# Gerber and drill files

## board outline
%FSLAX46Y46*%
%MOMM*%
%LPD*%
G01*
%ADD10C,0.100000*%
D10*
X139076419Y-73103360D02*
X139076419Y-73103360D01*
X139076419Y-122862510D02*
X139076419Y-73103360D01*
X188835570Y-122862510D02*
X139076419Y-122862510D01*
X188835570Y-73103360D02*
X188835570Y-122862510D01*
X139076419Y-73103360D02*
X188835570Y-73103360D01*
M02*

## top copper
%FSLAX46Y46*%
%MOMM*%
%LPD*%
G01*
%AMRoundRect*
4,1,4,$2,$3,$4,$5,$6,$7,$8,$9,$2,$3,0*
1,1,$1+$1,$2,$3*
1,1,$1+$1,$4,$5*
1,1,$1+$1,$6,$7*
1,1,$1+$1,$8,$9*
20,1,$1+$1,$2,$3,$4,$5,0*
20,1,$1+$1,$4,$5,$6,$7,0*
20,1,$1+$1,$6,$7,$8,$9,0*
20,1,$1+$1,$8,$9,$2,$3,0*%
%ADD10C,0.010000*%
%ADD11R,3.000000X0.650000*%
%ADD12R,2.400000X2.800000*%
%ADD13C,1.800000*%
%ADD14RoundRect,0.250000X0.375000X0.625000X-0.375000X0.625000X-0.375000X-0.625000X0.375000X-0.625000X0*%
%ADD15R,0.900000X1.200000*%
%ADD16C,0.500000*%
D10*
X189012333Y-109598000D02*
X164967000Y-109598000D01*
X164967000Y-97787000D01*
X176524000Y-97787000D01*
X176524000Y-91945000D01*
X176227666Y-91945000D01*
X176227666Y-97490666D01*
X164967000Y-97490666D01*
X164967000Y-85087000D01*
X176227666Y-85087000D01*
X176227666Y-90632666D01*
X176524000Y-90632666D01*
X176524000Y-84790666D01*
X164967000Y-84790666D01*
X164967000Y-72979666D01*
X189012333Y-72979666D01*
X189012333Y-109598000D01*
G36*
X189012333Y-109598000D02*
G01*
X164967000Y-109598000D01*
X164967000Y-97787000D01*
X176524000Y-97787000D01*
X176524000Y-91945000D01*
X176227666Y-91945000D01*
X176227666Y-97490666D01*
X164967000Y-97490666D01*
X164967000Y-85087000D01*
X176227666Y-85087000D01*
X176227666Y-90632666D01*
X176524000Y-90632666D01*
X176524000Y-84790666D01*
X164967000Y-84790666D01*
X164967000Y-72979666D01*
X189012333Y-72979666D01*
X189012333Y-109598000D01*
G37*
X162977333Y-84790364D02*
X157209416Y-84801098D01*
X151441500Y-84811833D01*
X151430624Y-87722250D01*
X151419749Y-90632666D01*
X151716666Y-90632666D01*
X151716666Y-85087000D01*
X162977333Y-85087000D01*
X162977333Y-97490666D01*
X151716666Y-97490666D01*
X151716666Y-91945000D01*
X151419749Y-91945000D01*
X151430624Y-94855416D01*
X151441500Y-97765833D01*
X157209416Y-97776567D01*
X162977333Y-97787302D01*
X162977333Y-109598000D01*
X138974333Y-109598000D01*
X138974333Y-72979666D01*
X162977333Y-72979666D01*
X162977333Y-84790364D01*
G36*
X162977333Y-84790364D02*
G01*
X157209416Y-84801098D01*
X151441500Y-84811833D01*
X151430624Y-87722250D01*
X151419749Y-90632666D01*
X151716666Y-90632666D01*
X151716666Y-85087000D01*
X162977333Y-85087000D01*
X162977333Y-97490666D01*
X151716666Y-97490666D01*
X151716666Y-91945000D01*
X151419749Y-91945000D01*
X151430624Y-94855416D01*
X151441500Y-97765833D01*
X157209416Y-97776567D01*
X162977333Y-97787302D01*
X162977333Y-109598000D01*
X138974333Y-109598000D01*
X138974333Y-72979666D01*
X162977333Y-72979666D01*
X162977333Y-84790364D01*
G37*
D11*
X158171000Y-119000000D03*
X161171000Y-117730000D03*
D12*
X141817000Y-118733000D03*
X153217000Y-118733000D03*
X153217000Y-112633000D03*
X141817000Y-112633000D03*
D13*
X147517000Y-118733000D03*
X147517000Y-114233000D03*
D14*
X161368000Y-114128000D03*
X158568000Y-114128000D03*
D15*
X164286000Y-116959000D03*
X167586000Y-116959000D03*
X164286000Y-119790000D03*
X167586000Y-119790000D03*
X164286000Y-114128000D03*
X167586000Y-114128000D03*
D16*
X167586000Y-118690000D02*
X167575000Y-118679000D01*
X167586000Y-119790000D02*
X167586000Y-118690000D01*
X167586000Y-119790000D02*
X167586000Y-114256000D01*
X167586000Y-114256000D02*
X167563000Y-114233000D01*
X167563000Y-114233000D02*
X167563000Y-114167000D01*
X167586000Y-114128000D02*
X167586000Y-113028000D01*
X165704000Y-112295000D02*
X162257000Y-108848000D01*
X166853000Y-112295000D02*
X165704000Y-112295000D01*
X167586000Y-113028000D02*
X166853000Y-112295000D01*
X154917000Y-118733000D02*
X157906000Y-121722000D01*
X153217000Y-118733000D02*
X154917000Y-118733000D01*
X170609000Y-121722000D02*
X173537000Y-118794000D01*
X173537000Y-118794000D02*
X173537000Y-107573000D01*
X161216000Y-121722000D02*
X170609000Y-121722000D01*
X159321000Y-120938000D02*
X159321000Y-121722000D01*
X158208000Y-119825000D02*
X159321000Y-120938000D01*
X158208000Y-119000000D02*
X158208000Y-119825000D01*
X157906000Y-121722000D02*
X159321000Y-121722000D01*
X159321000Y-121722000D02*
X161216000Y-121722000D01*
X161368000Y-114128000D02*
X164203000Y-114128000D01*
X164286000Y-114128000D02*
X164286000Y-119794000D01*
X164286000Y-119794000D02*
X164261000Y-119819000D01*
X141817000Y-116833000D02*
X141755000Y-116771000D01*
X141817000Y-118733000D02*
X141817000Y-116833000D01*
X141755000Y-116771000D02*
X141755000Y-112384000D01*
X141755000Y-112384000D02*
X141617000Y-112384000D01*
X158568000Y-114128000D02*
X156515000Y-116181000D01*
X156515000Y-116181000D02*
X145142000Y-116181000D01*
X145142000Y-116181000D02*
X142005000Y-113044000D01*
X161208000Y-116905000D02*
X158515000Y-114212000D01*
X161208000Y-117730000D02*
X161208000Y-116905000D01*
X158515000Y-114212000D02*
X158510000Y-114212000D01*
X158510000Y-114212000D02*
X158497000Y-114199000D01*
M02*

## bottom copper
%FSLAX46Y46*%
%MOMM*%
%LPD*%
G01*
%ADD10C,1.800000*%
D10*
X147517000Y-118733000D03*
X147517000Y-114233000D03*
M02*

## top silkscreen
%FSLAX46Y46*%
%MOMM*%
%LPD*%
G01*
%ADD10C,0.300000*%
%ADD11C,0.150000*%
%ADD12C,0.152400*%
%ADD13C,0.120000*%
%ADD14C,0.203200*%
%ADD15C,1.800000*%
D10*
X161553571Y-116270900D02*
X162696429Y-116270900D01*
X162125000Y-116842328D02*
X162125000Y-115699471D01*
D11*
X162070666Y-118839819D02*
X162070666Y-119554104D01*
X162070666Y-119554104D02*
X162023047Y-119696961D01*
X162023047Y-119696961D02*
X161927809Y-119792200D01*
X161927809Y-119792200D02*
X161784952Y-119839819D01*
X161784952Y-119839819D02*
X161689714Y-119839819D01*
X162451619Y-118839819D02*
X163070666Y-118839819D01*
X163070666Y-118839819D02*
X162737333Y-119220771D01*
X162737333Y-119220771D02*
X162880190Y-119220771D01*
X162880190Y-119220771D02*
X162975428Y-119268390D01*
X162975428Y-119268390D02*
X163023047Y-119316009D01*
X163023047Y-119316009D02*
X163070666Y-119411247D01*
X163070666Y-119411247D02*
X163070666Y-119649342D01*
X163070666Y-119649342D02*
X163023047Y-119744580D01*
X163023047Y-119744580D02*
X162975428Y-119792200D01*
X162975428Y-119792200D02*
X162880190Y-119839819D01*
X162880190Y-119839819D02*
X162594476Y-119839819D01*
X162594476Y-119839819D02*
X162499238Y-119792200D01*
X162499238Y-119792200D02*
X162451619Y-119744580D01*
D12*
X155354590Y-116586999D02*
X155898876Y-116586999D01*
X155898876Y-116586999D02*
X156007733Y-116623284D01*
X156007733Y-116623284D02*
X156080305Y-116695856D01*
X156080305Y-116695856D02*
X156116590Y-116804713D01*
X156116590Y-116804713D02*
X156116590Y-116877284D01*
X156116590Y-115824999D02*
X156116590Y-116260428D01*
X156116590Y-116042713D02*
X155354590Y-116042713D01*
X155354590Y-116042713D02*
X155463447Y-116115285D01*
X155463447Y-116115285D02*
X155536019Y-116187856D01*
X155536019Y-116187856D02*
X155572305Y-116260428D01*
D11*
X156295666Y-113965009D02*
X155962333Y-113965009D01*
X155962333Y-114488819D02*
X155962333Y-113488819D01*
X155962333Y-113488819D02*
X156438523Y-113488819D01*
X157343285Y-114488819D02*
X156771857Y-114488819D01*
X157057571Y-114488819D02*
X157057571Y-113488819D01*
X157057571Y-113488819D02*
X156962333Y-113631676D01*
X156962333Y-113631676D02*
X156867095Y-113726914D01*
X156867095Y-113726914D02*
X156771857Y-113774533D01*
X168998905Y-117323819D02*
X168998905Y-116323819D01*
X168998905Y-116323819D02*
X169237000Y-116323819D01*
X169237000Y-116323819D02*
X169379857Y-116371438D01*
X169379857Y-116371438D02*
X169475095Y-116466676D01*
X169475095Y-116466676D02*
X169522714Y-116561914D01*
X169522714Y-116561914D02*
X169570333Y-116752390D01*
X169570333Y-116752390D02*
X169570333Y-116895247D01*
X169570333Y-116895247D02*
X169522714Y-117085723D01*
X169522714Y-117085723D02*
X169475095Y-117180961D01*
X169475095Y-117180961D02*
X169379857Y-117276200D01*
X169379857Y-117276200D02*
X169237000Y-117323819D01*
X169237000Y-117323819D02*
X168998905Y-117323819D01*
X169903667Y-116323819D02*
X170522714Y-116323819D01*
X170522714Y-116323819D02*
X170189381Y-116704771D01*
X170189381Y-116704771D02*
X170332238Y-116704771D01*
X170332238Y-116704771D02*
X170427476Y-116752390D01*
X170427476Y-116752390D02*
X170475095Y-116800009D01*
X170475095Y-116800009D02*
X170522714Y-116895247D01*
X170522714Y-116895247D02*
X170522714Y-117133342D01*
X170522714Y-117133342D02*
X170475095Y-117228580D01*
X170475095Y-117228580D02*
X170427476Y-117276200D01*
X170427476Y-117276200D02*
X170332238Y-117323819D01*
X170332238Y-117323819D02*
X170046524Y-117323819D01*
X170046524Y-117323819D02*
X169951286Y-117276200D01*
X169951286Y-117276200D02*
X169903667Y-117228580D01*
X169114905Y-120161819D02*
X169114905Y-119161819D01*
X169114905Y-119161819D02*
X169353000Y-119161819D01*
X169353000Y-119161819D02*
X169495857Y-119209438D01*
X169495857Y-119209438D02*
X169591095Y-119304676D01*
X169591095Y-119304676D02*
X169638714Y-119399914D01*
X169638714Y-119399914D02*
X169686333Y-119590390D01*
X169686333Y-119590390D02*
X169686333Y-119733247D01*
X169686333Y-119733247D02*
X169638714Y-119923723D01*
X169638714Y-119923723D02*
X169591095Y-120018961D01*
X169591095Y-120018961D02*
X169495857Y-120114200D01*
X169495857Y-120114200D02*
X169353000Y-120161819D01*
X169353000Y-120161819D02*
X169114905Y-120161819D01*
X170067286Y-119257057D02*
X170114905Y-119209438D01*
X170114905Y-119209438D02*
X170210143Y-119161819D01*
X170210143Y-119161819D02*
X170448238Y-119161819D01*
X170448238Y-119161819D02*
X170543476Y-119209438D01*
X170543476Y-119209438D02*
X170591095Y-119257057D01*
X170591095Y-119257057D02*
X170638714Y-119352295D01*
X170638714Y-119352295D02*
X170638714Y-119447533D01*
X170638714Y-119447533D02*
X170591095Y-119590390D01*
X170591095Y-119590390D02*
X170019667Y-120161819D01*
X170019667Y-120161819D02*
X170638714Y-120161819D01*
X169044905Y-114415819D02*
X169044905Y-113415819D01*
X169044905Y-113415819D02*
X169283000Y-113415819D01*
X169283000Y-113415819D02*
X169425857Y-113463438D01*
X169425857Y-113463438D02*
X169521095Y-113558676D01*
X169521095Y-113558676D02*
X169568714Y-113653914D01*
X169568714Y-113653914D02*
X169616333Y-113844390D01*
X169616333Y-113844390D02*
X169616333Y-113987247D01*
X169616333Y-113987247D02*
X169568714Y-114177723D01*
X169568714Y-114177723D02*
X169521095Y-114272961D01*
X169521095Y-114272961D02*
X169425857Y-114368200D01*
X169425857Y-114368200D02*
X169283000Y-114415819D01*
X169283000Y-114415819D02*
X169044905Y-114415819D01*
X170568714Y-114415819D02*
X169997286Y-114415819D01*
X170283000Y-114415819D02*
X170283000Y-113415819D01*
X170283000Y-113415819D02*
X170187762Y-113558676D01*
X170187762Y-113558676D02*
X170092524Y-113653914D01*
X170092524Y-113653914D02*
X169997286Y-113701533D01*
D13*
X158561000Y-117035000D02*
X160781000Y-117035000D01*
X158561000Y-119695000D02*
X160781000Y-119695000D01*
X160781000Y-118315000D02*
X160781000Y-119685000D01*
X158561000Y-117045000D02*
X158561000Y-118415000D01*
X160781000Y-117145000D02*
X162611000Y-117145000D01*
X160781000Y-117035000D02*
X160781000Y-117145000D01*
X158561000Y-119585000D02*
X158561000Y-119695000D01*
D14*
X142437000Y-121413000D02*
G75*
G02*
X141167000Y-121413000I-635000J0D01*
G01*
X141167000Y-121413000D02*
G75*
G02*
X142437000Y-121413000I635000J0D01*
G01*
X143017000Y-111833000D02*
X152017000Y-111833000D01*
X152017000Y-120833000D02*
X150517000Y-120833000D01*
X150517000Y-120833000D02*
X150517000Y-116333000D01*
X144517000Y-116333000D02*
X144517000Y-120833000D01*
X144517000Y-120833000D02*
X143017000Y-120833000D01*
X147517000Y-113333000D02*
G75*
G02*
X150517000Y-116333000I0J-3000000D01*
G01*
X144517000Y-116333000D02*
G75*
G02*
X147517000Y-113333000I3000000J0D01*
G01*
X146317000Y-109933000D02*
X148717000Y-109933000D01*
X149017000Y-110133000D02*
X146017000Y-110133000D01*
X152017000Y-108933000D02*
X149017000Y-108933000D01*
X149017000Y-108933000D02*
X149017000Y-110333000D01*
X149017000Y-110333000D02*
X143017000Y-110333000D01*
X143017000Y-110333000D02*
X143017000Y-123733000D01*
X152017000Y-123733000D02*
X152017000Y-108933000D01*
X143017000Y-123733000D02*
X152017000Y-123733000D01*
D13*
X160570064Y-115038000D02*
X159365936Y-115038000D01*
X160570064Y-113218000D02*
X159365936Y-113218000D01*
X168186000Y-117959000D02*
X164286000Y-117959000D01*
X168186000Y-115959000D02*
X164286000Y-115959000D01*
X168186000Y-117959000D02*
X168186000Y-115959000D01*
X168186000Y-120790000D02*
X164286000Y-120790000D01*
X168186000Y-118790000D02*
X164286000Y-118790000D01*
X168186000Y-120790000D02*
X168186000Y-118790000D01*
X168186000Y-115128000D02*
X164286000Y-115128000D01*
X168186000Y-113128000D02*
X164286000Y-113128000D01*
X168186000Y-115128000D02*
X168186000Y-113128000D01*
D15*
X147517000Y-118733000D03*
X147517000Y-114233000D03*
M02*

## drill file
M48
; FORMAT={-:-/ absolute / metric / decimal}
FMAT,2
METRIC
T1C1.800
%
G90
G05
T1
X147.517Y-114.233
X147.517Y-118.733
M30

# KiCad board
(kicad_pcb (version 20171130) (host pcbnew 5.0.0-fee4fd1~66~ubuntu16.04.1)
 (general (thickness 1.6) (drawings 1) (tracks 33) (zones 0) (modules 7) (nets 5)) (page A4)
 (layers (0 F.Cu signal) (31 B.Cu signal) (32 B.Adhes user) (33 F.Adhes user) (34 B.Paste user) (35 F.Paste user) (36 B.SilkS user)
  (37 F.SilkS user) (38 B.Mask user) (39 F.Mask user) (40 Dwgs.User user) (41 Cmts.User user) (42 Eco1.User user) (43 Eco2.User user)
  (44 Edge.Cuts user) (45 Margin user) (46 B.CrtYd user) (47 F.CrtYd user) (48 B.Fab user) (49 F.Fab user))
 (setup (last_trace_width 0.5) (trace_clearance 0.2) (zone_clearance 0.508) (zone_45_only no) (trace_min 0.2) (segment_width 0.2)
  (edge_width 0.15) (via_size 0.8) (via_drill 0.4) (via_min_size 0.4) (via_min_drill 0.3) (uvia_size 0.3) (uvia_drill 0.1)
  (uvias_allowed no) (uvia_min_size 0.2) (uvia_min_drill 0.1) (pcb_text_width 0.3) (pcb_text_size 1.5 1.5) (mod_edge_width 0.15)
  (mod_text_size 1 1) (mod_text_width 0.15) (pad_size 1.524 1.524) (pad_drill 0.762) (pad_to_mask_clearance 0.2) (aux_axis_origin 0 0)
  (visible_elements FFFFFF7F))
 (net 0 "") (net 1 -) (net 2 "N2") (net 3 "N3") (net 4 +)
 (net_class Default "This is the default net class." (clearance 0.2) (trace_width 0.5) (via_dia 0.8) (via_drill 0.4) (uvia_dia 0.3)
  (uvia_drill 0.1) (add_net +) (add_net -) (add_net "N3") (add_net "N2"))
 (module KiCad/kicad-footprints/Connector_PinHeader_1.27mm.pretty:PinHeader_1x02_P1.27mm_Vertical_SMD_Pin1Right (layer F.Cu)
  (at 159.671 118.365)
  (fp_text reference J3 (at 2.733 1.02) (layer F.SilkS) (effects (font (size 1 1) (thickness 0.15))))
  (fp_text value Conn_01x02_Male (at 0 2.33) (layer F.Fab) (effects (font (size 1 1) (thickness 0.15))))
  (fp_line (start -1.11 -1.33) (end 1.11 -1.33) (layer F.SilkS) (width 0.12))
  (fp_line (start -1.11 1.33) (end 1.11 1.33) (layer F.SilkS) (width 0.12))
  (fp_line (start 1.11 -0.05) (end 1.11 1.32) (layer F.SilkS) (width 0.12))
  (fp_line (start -1.11 -1.32) (end -1.11 0.05) (layer F.SilkS) (width 0.12))
  (fp_line (start 1.11 -1.22) (end 2.94 -1.22) (layer F.SilkS) (width 0.12))
  (fp_line (start 1.11 -1.33) (end 1.11 -1.22) (layer F.SilkS) (width 0.12))
  (fp_line (start -1.11 1.22) (end -1.11 1.33) (layer F.SilkS) (width 0.12))
  (pad 2 smd rect (at -1.5 0.635) (size 3 0.65) (layers F.Cu F.Paste F.Mask) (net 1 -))
  (pad 1 smd rect (at 1.5 -0.635) (size 3 0.65) (layers F.Cu F.Paste F.Mask) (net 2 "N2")))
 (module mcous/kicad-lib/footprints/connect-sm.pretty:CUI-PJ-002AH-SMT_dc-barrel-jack (layer F.Cu) (at 147.517 116.333 90)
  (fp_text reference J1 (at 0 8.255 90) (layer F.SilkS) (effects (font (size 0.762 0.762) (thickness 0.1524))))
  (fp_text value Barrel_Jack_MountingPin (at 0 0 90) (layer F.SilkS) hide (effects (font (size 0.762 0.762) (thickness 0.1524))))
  (fp_circle (center -5.08 -5.715) (end -4.445 -5.715) (layer F.SilkS) (width 0.2032))
  (fp_line (start 4.5 -4.5) (end 4.5 4.5) (layer F.SilkS) (width 0.2032))
  (fp_line (start -4.5 4.5) (end -4.5 3) (layer F.SilkS) (width 0.2032))
  (fp_line (start -4.5 3) (end 0 3) (layer F.SilkS) (width 0.2032))
  (fp_line (start 0 -3) (end -4.5 -3) (layer F.SilkS) (width 0.2032))
  (fp_line (start -4.5 -3) (end -4.5 -4.5) (layer F.SilkS) (width 0.2032))
  (fp_arc (start 0 0) (end 3 0) (angle 90) (layer F.SilkS) (width 0.2032))
  (fp_arc (start 0 0) (end 0 -3) (angle 90) (layer F.SilkS) (width 0.2032))
  (fp_line (start 6.4 -1.2) (end 6.4 1.2) (layer F.SilkS) (width 0.2032))
  (fp_line (start 6.2 1.5) (end 6.2 -1.5) (layer F.SilkS) (width 0.2032))
  (fp_line (start 7.4 4.5) (end 7.4 1.5) (layer F.SilkS) (width 0.2032))
  (fp_line (start 7.4 1.5) (end 6 1.5) (layer F.SilkS) (width 0.2032))
  (fp_line (start 6 1.5) (end 6 -4.5) (layer F.SilkS) (width 0.2032))
  (fp_line (start 6 -4.5) (end -7.4 -4.5) (layer F.SilkS) (width 0.2032))
  (fp_line (start -7.4 4.5) (end 7.4 4.5) (layer F.SilkS) (width 0.2032))
  (fp_line (start -7.4 -4.5) (end -7.4 4.5) (layer F.SilkS) (width 0.2032))
  (pad 1 smd rect (at -2.4 -5.7 90) (size 2.8 2.4) (layers F.Cu F.Paste F.Mask) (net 2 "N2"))
  (pad 2 smd rect (at -2.4 5.7 90) (size 2.8 2.4) (layers F.Cu F.Paste F.Mask) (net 1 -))
  (pad 3 smd rect (at 3.7 5.7 90) (size 2.8 2.4) (layers F.Cu F.Paste F.Mask))
  (pad 1 smd rect (at 3.7 -5.7 90) (size 2.8 2.4) (layers F.Cu F.Paste F.Mask) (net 2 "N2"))
  (pad "" thru_hole circle (at -2.4 0 90) (size 1.8 1.8) (drill 1.8) (layers *.Cu *.Mask F.SilkS))
  (pad "" thru_hole circle (at 2.1 0 90) (size 1.8 1.8) (drill 1.8) (layers *.Cu *.Mask F.SilkS)))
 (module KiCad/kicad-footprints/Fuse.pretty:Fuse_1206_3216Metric (layer F.Cu) (at 159.968 114.128 180)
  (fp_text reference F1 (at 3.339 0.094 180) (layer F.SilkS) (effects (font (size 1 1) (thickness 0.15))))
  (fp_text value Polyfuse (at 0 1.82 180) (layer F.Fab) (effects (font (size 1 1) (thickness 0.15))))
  (fp_line (start -0.602064 -0.91) (end 0.602064 -0.91) (layer F.SilkS) (width 0.12))
  (fp_line (start -0.602064 0.91) (end 0.602064 0.91) (layer F.SilkS) (width 0.12))
  (pad 1 smd roundrect (at -1.4 0 180) (size 1.25 1.75) (layers F.Cu F.Paste F.Mask) (roundrect_rratio 0.2) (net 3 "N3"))
  (pad 2 smd roundrect (at 1.4 0 180) (size 1.25 1.75) (layers F.Cu F.Paste F.Mask) (roundrect_rratio 0.2) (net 2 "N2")))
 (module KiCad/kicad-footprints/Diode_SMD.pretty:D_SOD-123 (layer F.Cu) (at 165.936 116.959 180)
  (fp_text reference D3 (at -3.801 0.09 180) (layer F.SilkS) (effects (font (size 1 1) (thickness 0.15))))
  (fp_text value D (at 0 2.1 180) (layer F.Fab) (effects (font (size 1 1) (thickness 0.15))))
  (fp_line (start -2.25 -1) (end 1.65 -1) (layer F.SilkS) (width 0.12))
  (fp_line (start -2.25 1) (end 1.65 1) (layer F.SilkS) (width 0.12))
  (fp_line (start -2.25 -1) (end -2.25 1) (layer F.SilkS) (width 0.12))
  (pad 2 smd rect (at 1.65 0 180) (size 0.9 1.2) (layers F.Cu F.Paste F.Mask) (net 3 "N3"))
  (pad 1 smd rect (at -1.65 0 180) (size 0.9 1.2) (layers F.Cu F.Paste F.Mask) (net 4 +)))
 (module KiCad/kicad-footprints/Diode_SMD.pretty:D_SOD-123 (layer F.Cu) (at 165.936 119.79 180)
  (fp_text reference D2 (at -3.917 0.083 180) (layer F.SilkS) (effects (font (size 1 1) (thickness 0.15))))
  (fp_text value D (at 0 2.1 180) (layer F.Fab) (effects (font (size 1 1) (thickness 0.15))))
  (fp_line (start -2.25 -1) (end 1.65 -1) (layer F.SilkS) (width 0.12))
  (fp_line (start -2.25 1) (end 1.65 1) (layer F.SilkS) (width 0.12))
  (fp_line (start -2.25 -1) (end -2.25 1) (layer F.SilkS) (width 0.12))
  (pad 2 smd rect (at 1.65 0 180) (size 0.9 1.2) (layers F.Cu F.Paste F.Mask) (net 3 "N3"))
  (pad 1 smd rect (at -1.65 0 180) (size 0.9 1.2) (layers F.Cu F.Paste F.Mask) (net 4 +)))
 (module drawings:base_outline (layer F.Cu) (at 175.254 80.007)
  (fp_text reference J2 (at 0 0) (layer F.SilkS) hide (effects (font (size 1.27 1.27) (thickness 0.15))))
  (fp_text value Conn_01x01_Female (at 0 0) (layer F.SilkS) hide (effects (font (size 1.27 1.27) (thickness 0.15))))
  (fp_line (start -36.177581 -6.90364) (end -36.177581 -6.90364) (layer Edge.Cuts) (width 0.1))
  (fp_line (start -36.177581 42.85551) (end -36.177581 -6.90364) (layer Edge.Cuts) (width 0.1))
  (fp_line (start 13.58157 42.85551) (end -36.177581 42.85551) (layer Edge.Cuts) (width 0.1))
  (fp_line (start 13.58157 -6.90364) (end 13.58157 42.85551) (layer Edge.Cuts) (width 0.1))
  (fp_line (start -36.177581 -6.90364) (end 13.58157 -6.90364) (layer Edge.Cuts) (width 0.1))
  (fp_poly
   (pts (xy 13.758333 29.591) (xy -10.287 29.591) (xy -10.287 17.78) (xy 1.27 17.78) (xy 1.27 11.938) (xy 0.973666 11.938)
    (xy 0.973666 17.483666) (xy -10.287 17.483666) (xy -10.287 5.08) (xy 0.973666 5.08) (xy 0.973666 10.625666) (xy 1.27 10.625666)
    (xy 1.27 4.783666) (xy -10.287 4.783666) (xy -10.287 -7.027334) (xy 13.758333 -7.027334) (xy 13.758333 29.591))
   (layer F.Cu) (width 0.01))
  (fp_poly
   (pts (xy -12.276667 4.783364) (xy -18.044584 4.794098) (xy -23.8125 4.804833) (xy -23.823376 7.71525) (xy -23.834251 10.625666)
    (xy -23.537334 10.625666) (xy -23.537334 5.08) (xy -12.276667 5.08) (xy -12.276667 17.483666) (xy -23.537334 17.483666)
    (xy -23.537334 11.938) (xy -23.834251 11.938) (xy -23.823376 14.848416) (xy -23.8125 17.758833) (xy -18.044584 17.769567)
    (xy -12.276667 17.780302) (xy -12.276667 29.591) (xy -36.279667 29.591) (xy -36.279667 -7.027334) (xy -12.276667 -7.027334)
    (xy -12.276667 4.783364))
   (layer F.Cu) (width 0.01)))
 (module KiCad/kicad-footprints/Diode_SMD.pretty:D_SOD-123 (layer F.Cu) (at 165.936 114.128 180)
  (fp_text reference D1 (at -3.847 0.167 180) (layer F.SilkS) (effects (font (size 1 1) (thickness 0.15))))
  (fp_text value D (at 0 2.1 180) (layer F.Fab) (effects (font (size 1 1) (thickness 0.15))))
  (fp_line (start -2.25 -1) (end 1.65 -1) (layer F.SilkS) (width 0.12))
  (fp_line (start -2.25 1) (end 1.65 1) (layer F.SilkS) (width 0.12))
  (fp_line (start -2.25 -1) (end -2.25 1) (layer F.SilkS) (width 0.12))
  (pad 2 smd rect (at 1.65 0 180) (size 0.9 1.2) (layers F.Cu F.Paste F.Mask) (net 3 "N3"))
  (pad 1 smd rect (at -1.65 0 180) (size 0.9 1.2) (layers F.Cu F.Paste F.Mask) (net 4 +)))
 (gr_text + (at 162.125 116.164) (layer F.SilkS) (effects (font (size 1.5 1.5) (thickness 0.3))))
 (segment (start 167.586 118.69) (end 167.575 118.679) (width 0.5) (layer F.Cu) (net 4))
 (segment (start 167.586 119.79) (end 167.586 118.69) (width 0.5) (layer F.Cu) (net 4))
 (segment (start 167.586 119.79) (end 167.586 114.256) (width 0.5) (layer F.Cu) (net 4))
 (segment (start 167.586 114.256) (end 167.563 114.233) (width 0.5) (layer F.Cu) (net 4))
 (segment (start 167.563 114.233) (end 167.563 114.167) (width 0.5) (layer F.Cu) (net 4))
 (segment (start 167.586 114.128) (end 167.586 113.028) (width 0.5) (layer F.Cu) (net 4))
 (segment (start 165.704 112.295) (end 162.257 108.848) (width 0.5) (layer F.Cu) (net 4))
 (segment (start 166.853 112.295) (end 165.704 112.295) (width 0.5) (layer F.Cu) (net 4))
 (segment (start 167.586 113.028) (end 166.853 112.295) (width 0.5) (layer F.Cu) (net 4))
 (segment (start 154.917 118.733) (end 157.906 121.722) (width 0.5) (layer F.Cu) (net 1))
 (segment (start 153.217 118.733) (end 154.917 118.733) (width 0.5) (layer F.Cu) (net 1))
 (segment (start 170.609 121.722) (end 173.537 118.794) (width 0.5) (layer F.Cu) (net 1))
 (segment (start 173.537 118.794) (end 173.537 107.573) (width 0.5) (layer F.Cu) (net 1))
 (segment (start 161.216 121.722) (end 170.609 121.722) (width 0.5) (layer F.Cu) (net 1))
 (segment (start 159.321 120.938) (end 159.321 121.722) (width 0.5) (layer F.Cu) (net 1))
 (segment (start 158.208 119.825) (end 159.321 120.938) (width 0.5) (layer F.Cu) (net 1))
 (segment (start 158.208 119) (end 158.208 119.825) (width 0.5) (layer F.Cu) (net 1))
 (segment (start 157.906 121.722) (end 159.321 121.722) (width 0.5) (layer F.Cu) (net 1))
 (segment (start 159.321 121.722) (end 161.216 121.722) (width 0.5) (layer F.Cu) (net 1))
 (segment (start 161.368 114.128) (end 164.203 114.128) (width 0.5) (layer F.Cu) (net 3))
 (segment (start 164.286 114.128) (end 164.286 119.794) (width 0.5) (layer F.Cu) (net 3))
 (segment (start 164.286 119.794) (end 164.261 119.819) (width 0.5) (layer F.Cu) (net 3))
 (segment (start 141.817 116.833) (end 141.755 116.771) (width 0.5) (layer F.Cu) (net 2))
 (segment (start 141.817 118.733) (end 141.817 116.833) (width 0.5) (layer F.Cu) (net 2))
 (segment (start 141.755 116.771) (end 141.755 112.384) (width 0.5) (layer F.Cu) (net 2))
 (segment (start 141.755 112.384) (end 141.617 112.384) (width 0.5) (layer F.Cu) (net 2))
 (segment (start 158.568 114.128) (end 156.515 116.181) (width 0.5) (layer F.Cu) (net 2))
 (segment (start 156.515 116.181) (end 145.142 116.181) (width 0.5) (layer F.Cu) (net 2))
 (segment (start 145.142 116.181) (end 142.005 113.044) (width 0.5) (layer F.Cu) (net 2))
 (segment (start 161.208 116.905) (end 158.515 114.212) (width 0.5) (layer F.Cu) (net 2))
 (segment (start 161.208 117.73) (end 161.208 116.905) (width 0.5) (layer F.Cu) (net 2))
 (segment (start 158.515 114.212) (end 158.51 114.212) (width 0.5) (layer F.Cu) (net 2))
 (segment (start 158.51 114.212) (end 158.497 114.199) (width 0.5) (layer F.Cu) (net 2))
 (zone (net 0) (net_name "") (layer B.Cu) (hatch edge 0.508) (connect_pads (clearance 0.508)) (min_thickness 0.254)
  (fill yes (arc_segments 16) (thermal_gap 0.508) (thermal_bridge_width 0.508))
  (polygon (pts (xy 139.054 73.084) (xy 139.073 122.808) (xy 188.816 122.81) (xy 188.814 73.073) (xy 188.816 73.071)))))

